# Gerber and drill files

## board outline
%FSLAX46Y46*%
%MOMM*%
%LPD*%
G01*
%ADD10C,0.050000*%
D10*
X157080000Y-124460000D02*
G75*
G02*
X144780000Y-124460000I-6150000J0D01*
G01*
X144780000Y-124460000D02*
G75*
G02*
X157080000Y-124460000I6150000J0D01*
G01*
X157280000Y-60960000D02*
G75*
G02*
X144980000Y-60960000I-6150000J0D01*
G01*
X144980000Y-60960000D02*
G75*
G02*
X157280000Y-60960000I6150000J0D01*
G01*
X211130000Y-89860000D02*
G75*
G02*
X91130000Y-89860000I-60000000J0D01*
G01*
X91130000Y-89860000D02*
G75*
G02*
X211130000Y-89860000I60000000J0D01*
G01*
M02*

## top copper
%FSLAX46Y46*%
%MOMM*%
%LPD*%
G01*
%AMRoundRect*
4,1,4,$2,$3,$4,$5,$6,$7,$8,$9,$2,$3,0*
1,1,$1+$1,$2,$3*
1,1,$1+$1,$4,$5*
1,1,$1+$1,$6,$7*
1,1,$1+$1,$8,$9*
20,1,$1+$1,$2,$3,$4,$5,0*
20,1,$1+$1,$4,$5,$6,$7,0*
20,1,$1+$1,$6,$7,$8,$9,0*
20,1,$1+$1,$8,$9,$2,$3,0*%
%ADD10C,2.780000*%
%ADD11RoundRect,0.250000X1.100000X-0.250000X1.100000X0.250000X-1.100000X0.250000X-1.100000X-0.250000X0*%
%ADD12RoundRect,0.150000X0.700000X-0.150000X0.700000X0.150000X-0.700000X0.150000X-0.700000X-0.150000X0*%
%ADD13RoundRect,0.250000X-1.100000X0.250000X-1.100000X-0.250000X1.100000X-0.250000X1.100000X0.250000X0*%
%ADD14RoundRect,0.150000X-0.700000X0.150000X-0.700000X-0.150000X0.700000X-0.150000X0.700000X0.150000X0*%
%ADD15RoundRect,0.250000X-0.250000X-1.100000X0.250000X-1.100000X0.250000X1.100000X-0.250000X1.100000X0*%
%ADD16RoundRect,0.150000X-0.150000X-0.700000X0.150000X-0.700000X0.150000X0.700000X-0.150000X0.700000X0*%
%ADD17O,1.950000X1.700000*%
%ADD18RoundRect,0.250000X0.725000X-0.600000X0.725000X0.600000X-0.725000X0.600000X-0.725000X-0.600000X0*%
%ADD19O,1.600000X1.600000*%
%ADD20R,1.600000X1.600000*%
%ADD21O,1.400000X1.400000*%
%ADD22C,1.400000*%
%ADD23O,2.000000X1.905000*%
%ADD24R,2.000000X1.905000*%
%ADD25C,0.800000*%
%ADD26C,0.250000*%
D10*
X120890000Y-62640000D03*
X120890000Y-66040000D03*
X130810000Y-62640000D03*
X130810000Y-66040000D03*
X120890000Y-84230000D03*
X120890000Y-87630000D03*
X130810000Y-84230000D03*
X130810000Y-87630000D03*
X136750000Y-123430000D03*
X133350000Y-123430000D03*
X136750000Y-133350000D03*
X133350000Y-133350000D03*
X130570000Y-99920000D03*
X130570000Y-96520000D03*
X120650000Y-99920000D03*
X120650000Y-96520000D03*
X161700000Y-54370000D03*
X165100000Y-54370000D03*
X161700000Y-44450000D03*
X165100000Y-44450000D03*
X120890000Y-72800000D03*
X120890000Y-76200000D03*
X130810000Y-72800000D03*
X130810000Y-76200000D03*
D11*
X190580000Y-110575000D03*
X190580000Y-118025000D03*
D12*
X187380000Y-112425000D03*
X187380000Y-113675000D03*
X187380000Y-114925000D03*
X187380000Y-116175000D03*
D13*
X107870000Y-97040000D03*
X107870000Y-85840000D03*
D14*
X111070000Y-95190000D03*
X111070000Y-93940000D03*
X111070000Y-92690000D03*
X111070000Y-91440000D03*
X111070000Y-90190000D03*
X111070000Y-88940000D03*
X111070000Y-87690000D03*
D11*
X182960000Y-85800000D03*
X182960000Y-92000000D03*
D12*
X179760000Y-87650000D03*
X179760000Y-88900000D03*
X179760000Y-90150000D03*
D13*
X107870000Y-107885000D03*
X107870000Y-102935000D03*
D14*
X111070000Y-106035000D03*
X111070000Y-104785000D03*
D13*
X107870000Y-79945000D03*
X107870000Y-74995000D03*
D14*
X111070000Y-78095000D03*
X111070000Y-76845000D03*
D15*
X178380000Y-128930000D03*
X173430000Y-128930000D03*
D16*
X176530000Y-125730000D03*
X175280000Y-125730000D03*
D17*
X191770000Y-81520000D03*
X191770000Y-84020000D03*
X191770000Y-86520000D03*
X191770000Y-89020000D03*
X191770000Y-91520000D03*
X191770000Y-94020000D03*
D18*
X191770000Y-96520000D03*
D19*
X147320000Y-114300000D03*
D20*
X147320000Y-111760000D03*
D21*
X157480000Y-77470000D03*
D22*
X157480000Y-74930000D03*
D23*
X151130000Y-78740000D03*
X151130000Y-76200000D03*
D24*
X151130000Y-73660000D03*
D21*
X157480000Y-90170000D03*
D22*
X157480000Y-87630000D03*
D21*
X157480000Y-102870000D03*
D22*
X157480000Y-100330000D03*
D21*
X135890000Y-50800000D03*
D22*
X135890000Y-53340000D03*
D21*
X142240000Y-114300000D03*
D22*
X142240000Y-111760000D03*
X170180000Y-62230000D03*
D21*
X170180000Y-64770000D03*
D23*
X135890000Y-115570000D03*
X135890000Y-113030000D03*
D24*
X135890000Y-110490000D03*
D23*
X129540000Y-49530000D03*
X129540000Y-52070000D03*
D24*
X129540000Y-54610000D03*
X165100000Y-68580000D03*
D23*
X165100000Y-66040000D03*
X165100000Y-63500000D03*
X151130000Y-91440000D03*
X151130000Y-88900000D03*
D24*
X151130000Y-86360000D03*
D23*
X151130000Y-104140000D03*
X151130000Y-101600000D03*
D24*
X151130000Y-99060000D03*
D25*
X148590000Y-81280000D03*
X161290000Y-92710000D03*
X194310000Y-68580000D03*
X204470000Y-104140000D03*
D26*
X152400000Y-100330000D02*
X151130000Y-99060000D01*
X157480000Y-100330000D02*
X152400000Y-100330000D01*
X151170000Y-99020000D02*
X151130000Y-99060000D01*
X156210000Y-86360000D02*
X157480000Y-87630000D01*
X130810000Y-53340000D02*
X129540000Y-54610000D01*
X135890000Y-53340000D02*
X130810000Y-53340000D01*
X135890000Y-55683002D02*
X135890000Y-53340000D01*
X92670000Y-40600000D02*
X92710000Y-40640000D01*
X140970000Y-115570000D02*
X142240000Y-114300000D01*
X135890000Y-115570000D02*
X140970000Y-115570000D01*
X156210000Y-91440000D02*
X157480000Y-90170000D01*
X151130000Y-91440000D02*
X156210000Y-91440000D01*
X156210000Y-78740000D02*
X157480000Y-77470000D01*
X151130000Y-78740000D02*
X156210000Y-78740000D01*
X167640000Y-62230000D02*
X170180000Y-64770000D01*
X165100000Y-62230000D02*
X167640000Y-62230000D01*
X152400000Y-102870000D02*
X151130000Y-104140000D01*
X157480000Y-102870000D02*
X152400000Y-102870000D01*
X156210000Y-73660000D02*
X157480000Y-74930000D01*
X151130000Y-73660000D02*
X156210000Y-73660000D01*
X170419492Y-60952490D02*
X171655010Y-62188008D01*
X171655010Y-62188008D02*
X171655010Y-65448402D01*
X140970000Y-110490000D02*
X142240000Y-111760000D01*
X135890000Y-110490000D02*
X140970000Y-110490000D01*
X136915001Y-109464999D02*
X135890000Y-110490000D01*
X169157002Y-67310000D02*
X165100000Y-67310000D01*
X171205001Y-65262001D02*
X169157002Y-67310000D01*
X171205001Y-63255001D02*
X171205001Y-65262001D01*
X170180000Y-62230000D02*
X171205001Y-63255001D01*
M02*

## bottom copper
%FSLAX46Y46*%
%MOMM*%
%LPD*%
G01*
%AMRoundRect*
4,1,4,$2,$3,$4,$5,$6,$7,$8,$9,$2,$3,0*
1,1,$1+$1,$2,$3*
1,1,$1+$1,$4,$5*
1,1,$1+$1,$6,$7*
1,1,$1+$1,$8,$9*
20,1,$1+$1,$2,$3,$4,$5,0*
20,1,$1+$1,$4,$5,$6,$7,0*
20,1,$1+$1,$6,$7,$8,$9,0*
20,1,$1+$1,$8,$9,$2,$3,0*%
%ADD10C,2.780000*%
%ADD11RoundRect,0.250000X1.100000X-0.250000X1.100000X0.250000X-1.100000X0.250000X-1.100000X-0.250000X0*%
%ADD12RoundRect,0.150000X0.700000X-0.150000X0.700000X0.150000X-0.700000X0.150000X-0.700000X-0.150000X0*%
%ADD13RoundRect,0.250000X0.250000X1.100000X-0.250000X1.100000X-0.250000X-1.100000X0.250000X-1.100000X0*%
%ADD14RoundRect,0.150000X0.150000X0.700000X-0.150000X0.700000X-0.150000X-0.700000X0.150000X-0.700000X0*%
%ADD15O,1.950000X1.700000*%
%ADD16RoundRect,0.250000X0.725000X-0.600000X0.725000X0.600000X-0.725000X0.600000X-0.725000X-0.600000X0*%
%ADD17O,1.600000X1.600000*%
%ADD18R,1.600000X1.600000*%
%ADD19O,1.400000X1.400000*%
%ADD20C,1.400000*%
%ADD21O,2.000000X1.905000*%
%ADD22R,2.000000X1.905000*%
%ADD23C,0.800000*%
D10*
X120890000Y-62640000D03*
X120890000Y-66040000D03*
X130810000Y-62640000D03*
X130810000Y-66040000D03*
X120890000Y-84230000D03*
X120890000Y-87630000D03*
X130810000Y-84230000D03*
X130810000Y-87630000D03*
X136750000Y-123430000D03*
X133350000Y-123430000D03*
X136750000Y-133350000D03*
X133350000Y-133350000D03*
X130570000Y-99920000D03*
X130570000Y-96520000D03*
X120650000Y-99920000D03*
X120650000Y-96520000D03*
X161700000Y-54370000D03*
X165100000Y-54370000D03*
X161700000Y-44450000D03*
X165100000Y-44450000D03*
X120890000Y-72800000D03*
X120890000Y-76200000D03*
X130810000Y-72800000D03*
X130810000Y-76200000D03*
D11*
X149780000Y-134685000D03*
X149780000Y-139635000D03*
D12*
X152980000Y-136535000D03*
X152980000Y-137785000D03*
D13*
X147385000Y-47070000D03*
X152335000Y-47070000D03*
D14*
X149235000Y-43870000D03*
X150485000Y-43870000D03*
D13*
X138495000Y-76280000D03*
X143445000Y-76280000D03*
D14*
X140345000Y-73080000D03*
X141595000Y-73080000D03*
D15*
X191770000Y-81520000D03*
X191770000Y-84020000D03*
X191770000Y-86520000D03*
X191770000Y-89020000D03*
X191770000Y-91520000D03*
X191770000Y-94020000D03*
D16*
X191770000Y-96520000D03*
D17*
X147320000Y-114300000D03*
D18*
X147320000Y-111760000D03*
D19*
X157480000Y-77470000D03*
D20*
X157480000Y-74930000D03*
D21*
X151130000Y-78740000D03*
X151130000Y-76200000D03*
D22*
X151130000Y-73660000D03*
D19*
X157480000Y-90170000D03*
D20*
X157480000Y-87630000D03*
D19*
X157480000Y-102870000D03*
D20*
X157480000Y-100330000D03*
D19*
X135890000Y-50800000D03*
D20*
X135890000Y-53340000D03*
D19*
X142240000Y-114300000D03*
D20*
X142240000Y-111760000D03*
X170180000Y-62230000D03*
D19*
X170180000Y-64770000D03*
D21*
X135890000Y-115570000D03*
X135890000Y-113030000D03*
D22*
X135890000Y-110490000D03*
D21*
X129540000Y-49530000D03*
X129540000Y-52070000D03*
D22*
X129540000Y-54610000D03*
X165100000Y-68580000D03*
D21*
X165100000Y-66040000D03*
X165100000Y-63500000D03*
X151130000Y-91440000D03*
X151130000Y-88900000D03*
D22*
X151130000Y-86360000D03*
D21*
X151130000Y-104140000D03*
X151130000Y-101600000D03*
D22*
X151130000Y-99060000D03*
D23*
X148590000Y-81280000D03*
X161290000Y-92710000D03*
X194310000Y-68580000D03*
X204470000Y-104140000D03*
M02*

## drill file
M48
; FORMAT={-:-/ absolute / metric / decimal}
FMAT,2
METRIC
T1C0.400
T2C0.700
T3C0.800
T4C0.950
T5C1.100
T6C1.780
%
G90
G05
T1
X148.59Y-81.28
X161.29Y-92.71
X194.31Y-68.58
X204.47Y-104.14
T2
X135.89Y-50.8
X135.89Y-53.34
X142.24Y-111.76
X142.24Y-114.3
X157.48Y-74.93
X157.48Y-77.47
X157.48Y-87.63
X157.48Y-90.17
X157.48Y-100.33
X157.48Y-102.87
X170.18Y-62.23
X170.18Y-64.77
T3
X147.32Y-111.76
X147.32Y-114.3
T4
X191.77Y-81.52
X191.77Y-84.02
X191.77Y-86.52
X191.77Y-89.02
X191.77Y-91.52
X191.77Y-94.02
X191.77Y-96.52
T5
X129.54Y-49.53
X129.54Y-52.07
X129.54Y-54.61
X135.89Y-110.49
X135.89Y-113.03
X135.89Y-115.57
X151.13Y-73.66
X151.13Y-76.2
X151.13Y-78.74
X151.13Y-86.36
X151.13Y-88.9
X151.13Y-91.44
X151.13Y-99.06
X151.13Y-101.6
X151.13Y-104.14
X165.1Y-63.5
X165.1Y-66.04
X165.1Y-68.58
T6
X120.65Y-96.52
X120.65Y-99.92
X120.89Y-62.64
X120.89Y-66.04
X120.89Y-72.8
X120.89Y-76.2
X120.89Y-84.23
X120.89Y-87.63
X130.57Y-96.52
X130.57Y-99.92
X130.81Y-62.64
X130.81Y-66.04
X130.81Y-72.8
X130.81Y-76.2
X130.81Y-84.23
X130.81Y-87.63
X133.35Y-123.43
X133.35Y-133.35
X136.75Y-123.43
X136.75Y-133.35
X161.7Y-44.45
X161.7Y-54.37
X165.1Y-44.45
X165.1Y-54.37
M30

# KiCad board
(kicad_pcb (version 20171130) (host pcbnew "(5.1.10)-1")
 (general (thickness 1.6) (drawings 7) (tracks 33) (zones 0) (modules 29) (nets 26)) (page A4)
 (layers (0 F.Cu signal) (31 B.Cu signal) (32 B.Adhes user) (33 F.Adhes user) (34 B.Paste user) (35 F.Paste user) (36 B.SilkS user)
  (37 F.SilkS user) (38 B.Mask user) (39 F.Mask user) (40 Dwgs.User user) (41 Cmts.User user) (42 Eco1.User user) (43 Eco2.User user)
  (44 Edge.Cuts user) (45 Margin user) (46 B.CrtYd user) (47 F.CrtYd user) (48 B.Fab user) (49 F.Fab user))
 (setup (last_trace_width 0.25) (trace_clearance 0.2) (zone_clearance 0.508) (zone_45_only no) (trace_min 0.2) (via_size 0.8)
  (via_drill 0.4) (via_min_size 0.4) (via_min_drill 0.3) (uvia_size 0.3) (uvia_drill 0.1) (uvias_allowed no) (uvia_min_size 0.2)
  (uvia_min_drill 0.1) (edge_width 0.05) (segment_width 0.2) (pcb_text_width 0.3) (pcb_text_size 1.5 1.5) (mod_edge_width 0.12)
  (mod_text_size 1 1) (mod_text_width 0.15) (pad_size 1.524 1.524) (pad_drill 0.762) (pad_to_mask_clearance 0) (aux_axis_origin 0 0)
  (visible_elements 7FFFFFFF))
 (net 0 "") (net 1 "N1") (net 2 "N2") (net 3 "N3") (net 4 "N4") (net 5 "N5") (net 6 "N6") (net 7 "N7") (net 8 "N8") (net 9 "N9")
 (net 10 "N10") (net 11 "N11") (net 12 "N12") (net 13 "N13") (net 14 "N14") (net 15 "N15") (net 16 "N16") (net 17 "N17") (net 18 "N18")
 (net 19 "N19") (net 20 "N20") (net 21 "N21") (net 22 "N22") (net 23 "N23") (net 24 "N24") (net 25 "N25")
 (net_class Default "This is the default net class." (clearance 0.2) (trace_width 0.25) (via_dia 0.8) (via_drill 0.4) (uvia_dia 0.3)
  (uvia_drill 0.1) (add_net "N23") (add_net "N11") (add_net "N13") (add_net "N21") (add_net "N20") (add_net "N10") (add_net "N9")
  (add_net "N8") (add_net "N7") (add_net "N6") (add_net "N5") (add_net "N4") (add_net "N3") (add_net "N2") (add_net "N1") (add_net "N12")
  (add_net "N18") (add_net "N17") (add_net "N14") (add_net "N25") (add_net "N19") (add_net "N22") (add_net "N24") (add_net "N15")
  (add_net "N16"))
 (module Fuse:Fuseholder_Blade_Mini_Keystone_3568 (layer F.Cu) (at 130.81 66.04 180)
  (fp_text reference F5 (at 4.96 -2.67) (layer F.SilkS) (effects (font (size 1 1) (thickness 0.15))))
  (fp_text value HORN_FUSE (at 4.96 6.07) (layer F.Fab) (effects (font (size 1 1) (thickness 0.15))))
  (pad 2 thru_hole circle (at 9.92 3.4 180) (size 2.78 2.78) (drill 1.78) (layers *.Cu *.Mask) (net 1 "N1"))
  (pad 2 thru_hole circle (at 9.92 0 180) (size 2.78 2.78) (drill 1.78) (layers *.Cu *.Mask) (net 1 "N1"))
  (pad 1 thru_hole circle (at 0 3.4 180) (size 2.78 2.78) (drill 1.78) (layers *.Cu *.Mask) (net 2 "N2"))
  (pad 1 thru_hole circle (at 0 0 180) (size 2.78 2.78) (drill 1.78) (layers *.Cu *.Mask) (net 2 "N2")))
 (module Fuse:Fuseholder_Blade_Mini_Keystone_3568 (layer F.Cu) (at 130.81 87.63 180)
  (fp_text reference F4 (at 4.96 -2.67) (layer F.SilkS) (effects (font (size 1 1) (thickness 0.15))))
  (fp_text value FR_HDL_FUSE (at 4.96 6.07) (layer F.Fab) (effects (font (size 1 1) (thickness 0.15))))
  (pad 2 thru_hole circle (at 9.92 3.4 180) (size 2.78 2.78) (drill 1.78) (layers *.Cu *.Mask) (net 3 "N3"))
  (pad 2 thru_hole circle (at 9.92 0 180) (size 2.78 2.78) (drill 1.78) (layers *.Cu *.Mask) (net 3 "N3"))
  (pad 1 thru_hole circle (at 0 3.4 180) (size 2.78 2.78) (drill 1.78) (layers *.Cu *.Mask) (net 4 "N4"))
  (pad 1 thru_hole circle (at 0 0 180) (size 2.78 2.78) (drill 1.78) (layers *.Cu *.Mask) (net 4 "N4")))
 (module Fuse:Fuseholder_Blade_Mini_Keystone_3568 (layer F.Cu) (at 133.35 133.35 90)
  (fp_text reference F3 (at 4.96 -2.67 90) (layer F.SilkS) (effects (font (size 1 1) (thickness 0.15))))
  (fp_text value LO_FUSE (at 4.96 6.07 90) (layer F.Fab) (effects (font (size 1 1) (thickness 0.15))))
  (pad 2 thru_hole circle (at 9.92 3.4 90) (size 2.78 2.78) (drill 1.78) (layers *.Cu *.Mask) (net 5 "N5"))
  (pad 2 thru_hole circle (at 9.92 0 90) (size 2.78 2.78) (drill 1.78) (layers *.Cu *.Mask) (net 5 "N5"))
  (pad 1 thru_hole circle (at 0 3.4 90) (size 2.78 2.78) (drill 1.78) (layers *.Cu *.Mask) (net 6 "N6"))
  (pad 1 thru_hole circle (at 0 0 90) (size 2.78 2.78) (drill 1.78) (layers *.Cu *.Mask) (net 6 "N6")))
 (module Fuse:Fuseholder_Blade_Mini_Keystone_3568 (layer F.Cu) (at 120.65 96.52)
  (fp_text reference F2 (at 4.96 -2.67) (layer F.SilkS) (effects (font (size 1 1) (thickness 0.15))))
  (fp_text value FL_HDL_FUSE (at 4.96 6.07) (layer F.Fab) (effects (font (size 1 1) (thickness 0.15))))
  (pad 2 thru_hole circle (at 9.92 3.4) (size 2.78 2.78) (drill 1.78) (layers *.Cu *.Mask) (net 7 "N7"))
  (pad 2 thru_hole circle (at 9.92 0) (size 2.78 2.78) (drill 1.78) (layers *.Cu *.Mask) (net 7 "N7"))
  (pad 1 thru_hole circle (at 0 3.4) (size 2.78 2.78) (drill 1.78) (layers *.Cu *.Mask) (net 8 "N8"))
  (pad 1 thru_hole circle (at 0 0) (size 2.78 2.78) (drill 1.78) (layers *.Cu *.Mask) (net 8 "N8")))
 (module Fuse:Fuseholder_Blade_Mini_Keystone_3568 (layer F.Cu) (at 165.1 44.45 270)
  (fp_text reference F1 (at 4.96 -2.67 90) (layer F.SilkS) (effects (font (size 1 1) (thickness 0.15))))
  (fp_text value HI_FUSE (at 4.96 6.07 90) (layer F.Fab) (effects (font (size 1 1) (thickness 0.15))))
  (pad 2 thru_hole circle (at 9.92 3.4 270) (size 2.78 2.78) (drill 1.78) (layers *.Cu *.Mask) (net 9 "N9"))
  (pad 2 thru_hole circle (at 9.92 0 270) (size 2.78 2.78) (drill 1.78) (layers *.Cu *.Mask) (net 9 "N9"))
  (pad 1 thru_hole circle (at 0 3.4 270) (size 2.78 2.78) (drill 1.78) (layers *.Cu *.Mask) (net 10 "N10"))
  (pad 1 thru_hole circle (at 0 0 270) (size 2.78 2.78) (drill 1.78) (layers *.Cu *.Mask) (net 10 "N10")))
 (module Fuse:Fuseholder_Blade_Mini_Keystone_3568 (layer F.Cu) (at 130.81 76.2 180)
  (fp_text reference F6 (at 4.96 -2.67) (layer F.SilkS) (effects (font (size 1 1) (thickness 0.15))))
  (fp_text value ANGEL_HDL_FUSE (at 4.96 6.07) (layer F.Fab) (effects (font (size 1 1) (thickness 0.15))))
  (pad 2 thru_hole circle (at 9.92 3.4 180) (size 2.78 2.78) (drill 1.78) (layers *.Cu *.Mask) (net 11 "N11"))
  (pad 2 thru_hole circle (at 9.92 0 180) (size 2.78 2.78) (drill 1.78) (layers *.Cu *.Mask) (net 11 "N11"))
  (pad 1 thru_hole circle (at 0 3.4 180) (size 2.78 2.78) (drill 1.78) (layers *.Cu *.Mask) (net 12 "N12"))
  (pad 1 thru_hole circle (at 0 0 180) (size 2.78 2.78) (drill 1.78) (layers *.Cu *.Mask) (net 12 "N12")))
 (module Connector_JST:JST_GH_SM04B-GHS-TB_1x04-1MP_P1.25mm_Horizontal (layer F.Cu) (at 189.23 114.3 90)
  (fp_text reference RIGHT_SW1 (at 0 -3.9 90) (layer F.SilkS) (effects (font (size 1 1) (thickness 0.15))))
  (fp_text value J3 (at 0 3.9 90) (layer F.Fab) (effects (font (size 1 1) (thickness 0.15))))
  (pad MP smd roundrect (at 3.725 1.35 90) (size 1 2.7) (layers F.Cu F.Paste F.Mask) (roundrect_rratio 0.25))
  (pad MP smd roundrect (at -3.725 1.35 90) (size 1 2.7) (layers F.Cu F.Paste F.Mask) (roundrect_rratio 0.25))
  (pad 4 smd roundrect (at 1.875 -1.85 90) (size 0.6 1.7) (layers F.Cu F.Paste F.Mask) (roundrect_rratio 0.25) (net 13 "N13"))
  (pad 3 smd roundrect (at 0.625 -1.85 90) (size 0.6 1.7) (layers F.Cu F.Paste F.Mask) (roundrect_rratio 0.25) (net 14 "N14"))
  (pad 2 smd roundrect (at -0.625 -1.85 90) (size 0.6 1.7) (layers F.Cu F.Paste F.Mask) (roundrect_rratio 0.25) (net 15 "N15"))
  (pad 1 smd roundrect (at -1.875 -1.85 90) (size 0.6 1.7) (layers F.Cu F.Paste F.Mask) (roundrect_rratio 0.25) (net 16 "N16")))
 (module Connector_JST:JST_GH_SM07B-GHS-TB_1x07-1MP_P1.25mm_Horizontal (layer F.Cu) (at 109.22 91.44 270)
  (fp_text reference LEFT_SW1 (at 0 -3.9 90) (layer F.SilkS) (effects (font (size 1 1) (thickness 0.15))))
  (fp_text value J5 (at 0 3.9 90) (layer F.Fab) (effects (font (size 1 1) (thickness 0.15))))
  (pad MP smd roundrect (at 5.6 1.35 270) (size 1 2.7) (layers F.Cu F.Paste F.Mask) (roundrect_rratio 0.25))
  (pad MP smd roundrect (at -5.6 1.35 270) (size 1 2.7) (layers F.Cu F.Paste F.Mask) (roundrect_rratio 0.25))
  (pad 7 smd roundrect (at 3.75 -1.85 270) (size 0.6 1.7) (layers F.Cu F.Paste F.Mask) (roundrect_rratio 0.25) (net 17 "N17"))
  (pad 6 smd roundrect (at 2.5 -1.85 270) (size 0.6 1.7) (layers F.Cu F.Paste F.Mask) (roundrect_rratio 0.25) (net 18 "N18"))
  (pad 5 smd roundrect (at 1.25 -1.85 270) (size 0.6 1.7) (layers F.Cu F.Paste F.Mask) (roundrect_rratio 0.25) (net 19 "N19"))
  (pad 4 smd roundrect (at 0 -1.85 270) (size 0.6 1.7) (layers F.Cu F.Paste F.Mask) (roundrect_rratio 0.25) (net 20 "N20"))
  (pad 3 smd roundrect (at -1.25 -1.85 270) (size 0.6 1.7) (layers F.Cu F.Paste F.Mask) (roundrect_rratio 0.25) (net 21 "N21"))
  (pad 2 smd roundrect (at -2.5 -1.85 270) (size 0.6 1.7) (layers F.Cu F.Paste F.Mask) (roundrect_rratio 0.25) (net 13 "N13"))
  (pad 1 smd roundrect (at -3.75 -1.85 270) (size 0.6 1.7) (layers F.Cu F.Paste F.Mask) (roundrect_rratio 0.25) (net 14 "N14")))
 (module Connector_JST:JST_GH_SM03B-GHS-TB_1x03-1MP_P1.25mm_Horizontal (layer F.Cu) (at 181.61 88.9 90)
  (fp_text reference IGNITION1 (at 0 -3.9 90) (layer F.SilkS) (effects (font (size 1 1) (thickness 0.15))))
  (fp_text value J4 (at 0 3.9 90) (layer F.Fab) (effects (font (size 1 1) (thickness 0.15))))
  (pad MP smd roundrect (at 3.1 1.35 90) (size 1 2.7) (layers F.Cu F.Paste F.Mask) (roundrect_rratio 0.25))
  (pad MP smd roundrect (at -3.1 1.35 90) (size 1 2.7) (layers F.Cu F.Paste F.Mask) (roundrect_rratio 0.25))
  (pad 3 smd roundrect (at 1.25 -1.85 90) (size 0.6 1.7) (layers F.Cu F.Paste F.Mask) (roundrect_rratio 0.25) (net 13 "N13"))
  (pad 2 smd roundrect (at 0 -1.85 90) (size 0.6 1.7) (layers F.Cu F.Paste F.Mask) (roundrect_rratio 0.25) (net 14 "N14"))
  (pad 1 smd roundrect (at -1.25 -1.85 90) (size 0.6 1.7) (layers F.Cu F.Paste F.Mask) (roundrect_rratio 0.25) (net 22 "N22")))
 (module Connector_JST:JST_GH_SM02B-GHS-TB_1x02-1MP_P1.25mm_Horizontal (layer F.Cu) (at 109.22 105.41 270)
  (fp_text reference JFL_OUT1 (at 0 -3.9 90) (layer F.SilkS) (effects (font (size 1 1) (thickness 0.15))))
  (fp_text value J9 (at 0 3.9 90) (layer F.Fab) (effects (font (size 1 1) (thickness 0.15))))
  (pad MP smd roundrect (at 2.475 1.35 270) (size 1 2.7) (layers F.Cu F.Paste F.Mask) (roundrect_rratio 0.25))
  (pad MP smd roundrect (at -2.475 1.35 270) (size 1 2.7) (layers F.Cu F.Paste F.Mask) (roundrect_rratio 0.25))
  (pad 2 smd roundrect (at 0.625 -1.85 270) (size 0.6 1.7) (layers F.Cu F.Paste F.Mask) (roundrect_rratio 0.25) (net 14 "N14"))
  (pad 1 smd roundrect (at -0.625 -1.85 270) (size 0.6 1.7) (layers F.Cu F.Paste F.Mask) (roundrect_rratio 0.25) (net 8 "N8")))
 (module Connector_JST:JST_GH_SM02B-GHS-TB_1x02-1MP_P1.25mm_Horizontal (layer B.Cu) (at 151.13 137.16 90)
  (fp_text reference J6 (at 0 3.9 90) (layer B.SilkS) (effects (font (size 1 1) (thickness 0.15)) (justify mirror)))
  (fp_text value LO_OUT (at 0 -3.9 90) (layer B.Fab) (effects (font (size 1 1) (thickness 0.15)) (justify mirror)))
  (pad MP smd roundrect (at 2.475 -1.35 90) (size 1 2.7) (layers B.Cu B.Paste B.Mask) (roundrect_rratio 0.25))
  (pad MP smd roundrect (at -2.475 -1.35 90) (size 1 2.7) (layers B.Cu B.Paste B.Mask) (roundrect_rratio 0.25))
  (pad 2 smd roundrect (at 0.625 1.85 90) (size 0.6 1.7) (layers B.Cu B.Paste B.Mask) (roundrect_rratio 0.25) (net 14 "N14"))
  (pad 1 smd roundrect (at -0.625 1.85 90) (size 0.6 1.7) (layers B.Cu B.Paste B.Mask) (roundrect_rratio 0.25) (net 6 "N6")))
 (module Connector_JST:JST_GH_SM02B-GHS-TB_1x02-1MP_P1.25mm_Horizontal (layer B.Cu) (at 149.86 45.72 180)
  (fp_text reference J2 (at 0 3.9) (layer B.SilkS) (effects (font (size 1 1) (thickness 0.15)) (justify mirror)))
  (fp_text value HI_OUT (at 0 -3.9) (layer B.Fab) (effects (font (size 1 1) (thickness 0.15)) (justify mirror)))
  (pad MP smd roundrect (at 2.475 -1.35 180) (size 1 2.7) (layers B.Cu B.Paste B.Mask) (roundrect_rratio 0.25))
  (pad MP smd roundrect (at -2.475 -1.35 180) (size 1 2.7) (layers B.Cu B.Paste B.Mask) (roundrect_rratio 0.25))
  (pad 2 smd roundrect (at 0.625 1.85 180) (size 0.6 1.7) (layers B.Cu B.Paste B.Mask) (roundrect_rratio 0.25) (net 14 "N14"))
  (pad 1 smd roundrect (at -0.625 1.85 180) (size 0.6 1.7) (layers B.Cu B.Paste B.Mask) (roundrect_rratio 0.25) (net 10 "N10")))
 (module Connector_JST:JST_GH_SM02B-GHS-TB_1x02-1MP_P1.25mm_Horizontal (layer F.Cu) (at 109.22 77.47 270)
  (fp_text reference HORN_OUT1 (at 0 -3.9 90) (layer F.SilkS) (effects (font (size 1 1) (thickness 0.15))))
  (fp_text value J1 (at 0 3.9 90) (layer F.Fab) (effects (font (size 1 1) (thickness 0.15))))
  (pad MP smd roundrect (at 2.475 1.35 270) (size 1 2.7) (layers F.Cu F.Paste F.Mask) (roundrect_rratio 0.25))
  (pad MP smd roundrect (at -2.475 1.35 270) (size 1 2.7) (layers F.Cu F.Paste F.Mask) (roundrect_rratio 0.25))
  (pad 2 smd roundrect (at 0.625 -1.85 270) (size 0.6 1.7) (layers F.Cu F.Paste F.Mask) (roundrect_rratio 0.25) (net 14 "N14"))
  (pad 1 smd roundrect (at -0.625 -1.85 270) (size 0.6 1.7) (layers F.Cu F.Paste F.Mask) (roundrect_rratio 0.25) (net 2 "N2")))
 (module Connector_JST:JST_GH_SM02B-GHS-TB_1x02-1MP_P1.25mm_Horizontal (layer B.Cu) (at 140.97 74.93 180)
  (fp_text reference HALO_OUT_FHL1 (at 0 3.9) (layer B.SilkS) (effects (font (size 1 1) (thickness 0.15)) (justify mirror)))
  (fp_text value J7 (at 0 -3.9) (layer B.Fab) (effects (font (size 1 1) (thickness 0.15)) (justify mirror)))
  (pad MP smd roundrect (at 2.475 -1.35 180) (size 1 2.7) (layers B.Cu B.Paste B.Mask) (roundrect_rratio 0.25))
  (pad MP smd roundrect (at -2.475 -1.35 180) (size 1 2.7) (layers B.Cu B.Paste B.Mask) (roundrect_rratio 0.25))
  (pad 2 smd roundrect (at 0.625 1.85 180) (size 0.6 1.7) (layers B.Cu B.Paste B.Mask) (roundrect_rratio 0.25) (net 14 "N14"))
  (pad 1 smd roundrect (at -0.625 1.85 180) (size 0.6 1.7) (layers B.Cu B.Paste B.Mask) (roundrect_rratio 0.25) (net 12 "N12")))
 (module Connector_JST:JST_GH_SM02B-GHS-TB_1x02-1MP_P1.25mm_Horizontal (layer F.Cu) (at 175.905 127.58)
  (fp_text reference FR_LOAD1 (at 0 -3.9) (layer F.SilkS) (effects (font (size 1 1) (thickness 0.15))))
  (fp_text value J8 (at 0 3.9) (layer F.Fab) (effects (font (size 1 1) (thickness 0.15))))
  (pad MP smd roundrect (at 2.475 1.35) (size 1 2.7) (layers F.Cu F.Paste F.Mask) (roundrect_rratio 0.25))
  (pad MP smd roundrect (at -2.475 1.35) (size 1 2.7) (layers F.Cu F.Paste F.Mask) (roundrect_rratio 0.25))
  (pad 2 smd roundrect (at 0.625 -1.85) (size 0.6 1.7) (layers F.Cu F.Paste F.Mask) (roundrect_rratio 0.25) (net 4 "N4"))
  (pad 1 smd roundrect (at -0.625 -1.85) (size 0.6 1.7) (layers F.Cu F.Paste F.Mask) (roundrect_rratio 0.25) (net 14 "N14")))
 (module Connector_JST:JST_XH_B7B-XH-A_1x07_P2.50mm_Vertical (layer F.Cu) (at 191.77 96.52 90)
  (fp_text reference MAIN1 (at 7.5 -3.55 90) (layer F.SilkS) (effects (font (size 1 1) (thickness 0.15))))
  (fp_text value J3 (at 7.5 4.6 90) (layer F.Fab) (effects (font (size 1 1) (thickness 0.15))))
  (pad 7 thru_hole oval (at 15 0 90) (size 1.7 1.95) (drill 0.95) (layers *.Cu *.Mask) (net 13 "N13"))
  (pad 6 thru_hole oval (at 12.5 0 90) (size 1.7 1.95) (drill 0.95) (layers *.Cu *.Mask) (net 22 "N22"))
  (pad 5 thru_hole oval (at 10 0 90) (size 1.7 1.95) (drill 0.95) (layers *.Cu *.Mask) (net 14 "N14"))
  (pad 4 thru_hole oval (at 7.5 0 90) (size 1.7 1.95) (drill 0.95) (layers *.Cu *.Mask) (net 18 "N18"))
  (pad 3 thru_hole oval (at 5 0 90) (size 1.7 1.95) (drill 0.95) (layers *.Cu *.Mask) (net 17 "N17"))
  (pad 2 thru_hole oval (at 2.5 0 90) (size 1.7 1.95) (drill 0.95) (layers *.Cu *.Mask) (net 16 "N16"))
  (pad 1 thru_hole roundrect (at 0 0 90) (size 1.7 1.95) (drill 0.95) (layers *.Cu *.Mask) (roundrect_rratio 0.147059) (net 15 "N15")))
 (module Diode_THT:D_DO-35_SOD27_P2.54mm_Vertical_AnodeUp (layer F.Cu) (at 147.32 111.76 270)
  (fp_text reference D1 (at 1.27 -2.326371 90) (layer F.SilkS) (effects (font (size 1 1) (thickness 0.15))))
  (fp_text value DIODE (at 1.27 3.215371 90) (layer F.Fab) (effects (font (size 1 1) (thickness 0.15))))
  (pad 2 thru_hole oval (at 2.54 0 270) (size 1.6 1.6) (drill 0.8) (layers *.Cu *.Mask) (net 20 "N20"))
  (pad 1 thru_hole rect (at 0 0 270) (size 1.6 1.6) (drill 0.8) (layers *.Cu *.Mask) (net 21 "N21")))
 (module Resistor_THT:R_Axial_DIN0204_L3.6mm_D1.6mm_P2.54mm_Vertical (layer F.Cu) (at 157.48 74.93 270)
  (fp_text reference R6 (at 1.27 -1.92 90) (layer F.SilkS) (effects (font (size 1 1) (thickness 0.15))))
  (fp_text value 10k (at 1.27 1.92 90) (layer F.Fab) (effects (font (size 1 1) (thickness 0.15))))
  (pad 2 thru_hole oval (at 2.54 0 270) (size 1.4 1.4) (drill 0.7) (layers *.Cu *.Mask) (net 13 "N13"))
  (pad 1 thru_hole circle (at 0 0 270) (size 1.4 1.4) (drill 0.7) (layers *.Cu *.Mask) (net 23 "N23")))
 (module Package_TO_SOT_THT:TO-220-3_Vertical (layer F.Cu) (at 151.13 73.66 270)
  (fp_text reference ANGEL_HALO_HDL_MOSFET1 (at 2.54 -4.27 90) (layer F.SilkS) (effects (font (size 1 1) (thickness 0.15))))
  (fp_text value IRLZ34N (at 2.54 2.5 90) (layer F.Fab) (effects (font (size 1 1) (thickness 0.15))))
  (pad 3 thru_hole oval (at 5.08 0 270) (size 1.905 2) (drill 1.1) (layers *.Cu *.Mask) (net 13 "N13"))
  (pad 2 thru_hole oval (at 2.54 0 270) (size 1.905 2) (drill 1.1) (layers *.Cu *.Mask) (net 11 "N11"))
  (pad 1 thru_hole rect (at 0 0 270) (size 1.905 2) (drill 1.1) (layers *.Cu *.Mask) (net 23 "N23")))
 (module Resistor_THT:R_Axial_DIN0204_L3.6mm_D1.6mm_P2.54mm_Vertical (layer F.Cu) (at 157.48 87.63 270)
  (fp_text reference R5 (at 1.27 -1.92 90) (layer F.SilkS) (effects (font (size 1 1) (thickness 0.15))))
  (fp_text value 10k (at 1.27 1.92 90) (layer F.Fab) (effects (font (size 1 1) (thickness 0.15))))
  (pad 2 thru_hole oval (at 2.54 0 270) (size 1.4 1.4) (drill 0.7) (layers *.Cu *.Mask) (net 13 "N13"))
  (pad 1 thru_hole circle (at 0 0 270) (size 1.4 1.4) (drill 0.7) (layers *.Cu *.Mask) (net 17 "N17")))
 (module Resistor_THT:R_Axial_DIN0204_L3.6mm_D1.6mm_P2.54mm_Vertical (layer F.Cu) (at 157.48 100.33 270)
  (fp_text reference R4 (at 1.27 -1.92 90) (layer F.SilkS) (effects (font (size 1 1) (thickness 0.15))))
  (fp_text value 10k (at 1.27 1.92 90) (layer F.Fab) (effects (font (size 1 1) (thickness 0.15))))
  (pad 2 thru_hole oval (at 2.54 0 270) (size 1.4 1.4) (drill 0.7) (layers *.Cu *.Mask) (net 13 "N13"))
  (pad 1 thru_hole circle (at 0 0 270) (size 1.4 1.4) (drill 0.7) (layers *.Cu *.Mask) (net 18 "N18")))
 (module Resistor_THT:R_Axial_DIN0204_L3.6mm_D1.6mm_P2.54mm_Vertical (layer F.Cu) (at 135.89 53.34 90)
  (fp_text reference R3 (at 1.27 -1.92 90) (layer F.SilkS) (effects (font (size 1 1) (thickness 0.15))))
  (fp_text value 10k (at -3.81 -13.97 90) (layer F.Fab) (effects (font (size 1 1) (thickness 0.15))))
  (pad 2 thru_hole oval (at 2.54 0 90) (size 1.4 1.4) (drill 0.7) (layers *.Cu *.Mask) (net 13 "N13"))
  (pad 1 thru_hole circle (at 0 0 90) (size 1.4 1.4) (drill 0.7) (layers *.Cu *.Mask) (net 19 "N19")))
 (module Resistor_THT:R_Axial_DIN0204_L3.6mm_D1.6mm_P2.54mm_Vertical (layer F.Cu) (at 142.24 111.76 270)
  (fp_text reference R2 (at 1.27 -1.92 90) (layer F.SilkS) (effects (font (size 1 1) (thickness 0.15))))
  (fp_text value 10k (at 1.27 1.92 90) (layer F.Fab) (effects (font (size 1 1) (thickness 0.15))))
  (pad 2 thru_hole oval (at 2.54 0 270) (size 1.4 1.4) (drill 0.7) (layers *.Cu *.Mask) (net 13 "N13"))
  (pad 1 thru_hole circle (at 0 0 270) (size 1.4 1.4) (drill 0.7) (layers *.Cu *.Mask) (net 20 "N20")))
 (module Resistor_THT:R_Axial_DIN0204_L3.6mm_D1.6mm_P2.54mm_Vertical (layer F.Cu) (at 170.18 62.23 270)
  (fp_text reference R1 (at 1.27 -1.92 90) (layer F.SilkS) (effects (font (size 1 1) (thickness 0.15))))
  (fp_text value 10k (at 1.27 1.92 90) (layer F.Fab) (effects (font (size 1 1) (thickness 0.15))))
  (pad 1 thru_hole circle (at 0 0 270) (size 1.4 1.4) (drill 0.7) (layers *.Cu *.Mask) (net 21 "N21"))
  (pad 2 thru_hole oval (at 2.54 0 270) (size 1.4 1.4) (drill 0.7) (layers *.Cu *.Mask) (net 13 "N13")))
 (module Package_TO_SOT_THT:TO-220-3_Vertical (layer F.Cu) (at 135.89 110.49 270)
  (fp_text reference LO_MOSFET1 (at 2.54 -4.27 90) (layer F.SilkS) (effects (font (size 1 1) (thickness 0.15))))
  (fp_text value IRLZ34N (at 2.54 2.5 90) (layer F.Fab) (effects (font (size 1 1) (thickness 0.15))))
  (pad 3 thru_hole oval (at 5.08 0 270) (size 1.905 2) (drill 1.1) (layers *.Cu *.Mask) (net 13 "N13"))
  (pad 2 thru_hole oval (at 2.54 0 270) (size 1.905 2) (drill 1.1) (layers *.Cu *.Mask) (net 5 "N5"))
  (pad 1 thru_hole rect (at 0 0 270) (size 1.905 2) (drill 1.1) (layers *.Cu *.Mask) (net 20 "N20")))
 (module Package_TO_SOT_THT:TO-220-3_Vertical (layer F.Cu) (at 129.54 54.61 90)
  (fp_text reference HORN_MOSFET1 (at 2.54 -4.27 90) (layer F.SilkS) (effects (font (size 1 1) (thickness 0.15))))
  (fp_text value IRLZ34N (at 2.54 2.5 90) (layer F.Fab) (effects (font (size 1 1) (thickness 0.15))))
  (pad 3 thru_hole oval (at 5.08 0 90) (size 1.905 2) (drill 1.1) (layers *.Cu *.Mask) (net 13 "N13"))
  (pad 2 thru_hole oval (at 2.54 0 90) (size 1.905 2) (drill 1.1) (layers *.Cu *.Mask) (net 1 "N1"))
  (pad 1 thru_hole rect (at 0 0 90) (size 1.905 2) (drill 1.1) (layers *.Cu *.Mask) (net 19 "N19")))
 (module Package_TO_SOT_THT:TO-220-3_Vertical (layer F.Cu) (at 165.1 68.58 90)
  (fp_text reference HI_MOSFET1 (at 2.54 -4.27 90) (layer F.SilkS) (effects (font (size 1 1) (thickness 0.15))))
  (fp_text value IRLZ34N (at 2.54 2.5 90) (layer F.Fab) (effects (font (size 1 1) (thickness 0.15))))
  (pad 1 thru_hole rect (at 0 0 90) (size 1.905 2) (drill 1.1) (layers *.Cu *.Mask) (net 21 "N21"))
  (pad 2 thru_hole oval (at 2.54 0 90) (size 1.905 2) (drill 1.1) (layers *.Cu *.Mask) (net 9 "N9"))
  (pad 3 thru_hole oval (at 5.08 0 90) (size 1.905 2) (drill 1.1) (layers *.Cu *.Mask) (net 13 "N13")))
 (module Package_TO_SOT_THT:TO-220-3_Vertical (layer F.Cu) (at 151.13 86.36 270)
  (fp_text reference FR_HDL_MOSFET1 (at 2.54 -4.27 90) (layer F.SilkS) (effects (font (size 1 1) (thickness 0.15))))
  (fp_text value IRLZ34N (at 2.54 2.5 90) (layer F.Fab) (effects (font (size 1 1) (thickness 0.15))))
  (pad 3 thru_hole oval (at 5.08 0 270) (size 1.905 2) (drill 1.1) (layers *.Cu *.Mask) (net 13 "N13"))
  (pad 2 thru_hole oval (at 2.54 0 270) (size 1.905 2) (drill 1.1) (layers *.Cu *.Mask) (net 3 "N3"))
  (pad 1 thru_hole rect (at 0 0 270) (size 1.905 2) (drill 1.1) (layers *.Cu *.Mask) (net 17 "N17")))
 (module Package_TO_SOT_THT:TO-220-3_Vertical (layer F.Cu) (at 151.13 99.06 270)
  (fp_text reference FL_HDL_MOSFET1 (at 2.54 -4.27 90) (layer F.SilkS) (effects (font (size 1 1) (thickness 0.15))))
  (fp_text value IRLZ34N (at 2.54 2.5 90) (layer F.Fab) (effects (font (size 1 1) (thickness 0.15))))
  (pad 3 thru_hole oval (at 5.08 0 270) (size 1.905 2) (drill 1.1) (layers *.Cu *.Mask) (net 13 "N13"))
  (pad 2 thru_hole oval (at 2.54 0 270) (size 1.905 2) (drill 1.1) (layers *.Cu *.Mask) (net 7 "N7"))
  (pad 1 thru_hole rect (at 0 0 270) (size 1.905 2) (drill 1.1) (layers *.Cu *.Mask) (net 18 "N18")))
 (gr_circle (center 150.93 124.46) (end 157.08 124.46) (layer Edge.Cuts) (width 0.05))
 (gr_circle (center 151.13 60.96) (end 157.28 60.96) (layer Edge.Cuts) (width 0.05))
 (gr_circle (center 151.13 89.86) (end 211.13 89.86) (layer Edge.Cuts) (width 0.05))
 (via (at 148.59 81.28) (size 0.8) (drill 0.4) (layers F.Cu B.Cu) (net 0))
 (segment (start 152.4 100.33) (end 151.13 99.06) (width 0.25) (layer F.Cu) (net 18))
 (segment (start 157.48 100.33) (end 152.4 100.33) (width 0.25) (layer F.Cu) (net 18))
 (segment (start 151.17 99.02) (end 151.13 99.06) (width 0.25) (layer F.Cu) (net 18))
 (segment (start 156.21 86.36) (end 157.48 87.63) (width 0.25) (layer F.Cu) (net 17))
 (via (at 161.29 92.71) (size 0.8) (drill 0.4) (layers F.Cu B.Cu) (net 1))
 (segment (start 130.81 53.34) (end 129.54 54.61) (width 0.25) (layer F.Cu) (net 19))
 (segment (start 135.89 53.34) (end 130.81 53.34) (width 0.25) (layer F.Cu) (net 19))
 (segment (start 135.89 55.683002) (end 135.89 53.34) (width 0.25) (layer F.Cu) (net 19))
 (via (at 194.31 68.58) (size 0.8) (drill 0.4) (layers F.Cu B.Cu) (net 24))
 (segment (start 92.67 40.6) (end 92.71 40.64) (width 0.25) (layer F.Cu) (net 2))
 (segment (start 140.97 115.57) (end 142.24 114.3) (width 0.25) (layer F.Cu) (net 13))
 (segment (start 135.89 115.57) (end 140.97 115.57) (width 0.25) (layer F.Cu) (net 13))
 (segment (start 156.21 91.44) (end 157.48 90.17) (width 0.25) (layer F.Cu) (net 13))
 (segment (start 151.13 91.44) (end 156.21 91.44) (width 0.25) (layer F.Cu) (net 13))
 (segment (start 156.21 78.74) (end 157.48 77.47) (width 0.25) (layer F.Cu) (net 13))
 (segment (start 151.13 78.74) (end 156.21 78.74) (width 0.25) (layer F.Cu) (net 13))
 (segment (start 167.64 62.23) (end 170.18 64.77) (width 0.25) (layer F.Cu) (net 13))
 (segment (start 165.1 62.23) (end 167.64 62.23) (width 0.25) (layer F.Cu) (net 13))
 (segment (start 152.4 102.87) (end 151.13 104.14) (width 0.25) (layer F.Cu) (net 13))
 (segment (start 157.48 102.87) (end 152.4 102.87) (width 0.25) (layer F.Cu) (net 13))
 (segment (start 156.21 73.66) (end 157.48 74.93) (width 0.25) (layer F.Cu) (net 23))
 (segment (start 151.13 73.66) (end 156.21 73.66) (width 0.25) (layer F.Cu) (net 23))
 (via (at 204.47 104.14) (size 0.8) (drill 0.4) (layers F.Cu B.Cu) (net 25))
 (segment (start 170.419492 60.95249) (end 171.65501 62.188008) (width 0.25) (layer F.Cu) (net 22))
 (segment (start 171.65501 62.188008) (end 171.65501 65.448402) (width 0.25) (layer F.Cu) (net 22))
 (segment (start 140.97 110.49) (end 142.24 111.76) (width 0.25) (layer F.Cu) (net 20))
 (segment (start 135.89 110.49) (end 140.97 110.49) (width 0.25) (layer F.Cu) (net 20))
 (segment (start 136.915001 109.464999) (end 135.89 110.49) (width 0.25) (layer F.Cu) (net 20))
 (segment (start 169.157002 67.31) (end 165.1 67.31) (width 0.25) (layer F.Cu) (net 21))
 (segment (start 171.205001 65.262001) (end 169.157002 67.31) (width 0.25) (layer F.Cu) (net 21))
 (segment (start 171.205001 63.255001) (end 171.205001 65.262001) (width 0.25) (layer F.Cu) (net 21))
 (segment (start 170.18 62.23) (end 171.205001 63.255001) (width 0.25) (layer F.Cu) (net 21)))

